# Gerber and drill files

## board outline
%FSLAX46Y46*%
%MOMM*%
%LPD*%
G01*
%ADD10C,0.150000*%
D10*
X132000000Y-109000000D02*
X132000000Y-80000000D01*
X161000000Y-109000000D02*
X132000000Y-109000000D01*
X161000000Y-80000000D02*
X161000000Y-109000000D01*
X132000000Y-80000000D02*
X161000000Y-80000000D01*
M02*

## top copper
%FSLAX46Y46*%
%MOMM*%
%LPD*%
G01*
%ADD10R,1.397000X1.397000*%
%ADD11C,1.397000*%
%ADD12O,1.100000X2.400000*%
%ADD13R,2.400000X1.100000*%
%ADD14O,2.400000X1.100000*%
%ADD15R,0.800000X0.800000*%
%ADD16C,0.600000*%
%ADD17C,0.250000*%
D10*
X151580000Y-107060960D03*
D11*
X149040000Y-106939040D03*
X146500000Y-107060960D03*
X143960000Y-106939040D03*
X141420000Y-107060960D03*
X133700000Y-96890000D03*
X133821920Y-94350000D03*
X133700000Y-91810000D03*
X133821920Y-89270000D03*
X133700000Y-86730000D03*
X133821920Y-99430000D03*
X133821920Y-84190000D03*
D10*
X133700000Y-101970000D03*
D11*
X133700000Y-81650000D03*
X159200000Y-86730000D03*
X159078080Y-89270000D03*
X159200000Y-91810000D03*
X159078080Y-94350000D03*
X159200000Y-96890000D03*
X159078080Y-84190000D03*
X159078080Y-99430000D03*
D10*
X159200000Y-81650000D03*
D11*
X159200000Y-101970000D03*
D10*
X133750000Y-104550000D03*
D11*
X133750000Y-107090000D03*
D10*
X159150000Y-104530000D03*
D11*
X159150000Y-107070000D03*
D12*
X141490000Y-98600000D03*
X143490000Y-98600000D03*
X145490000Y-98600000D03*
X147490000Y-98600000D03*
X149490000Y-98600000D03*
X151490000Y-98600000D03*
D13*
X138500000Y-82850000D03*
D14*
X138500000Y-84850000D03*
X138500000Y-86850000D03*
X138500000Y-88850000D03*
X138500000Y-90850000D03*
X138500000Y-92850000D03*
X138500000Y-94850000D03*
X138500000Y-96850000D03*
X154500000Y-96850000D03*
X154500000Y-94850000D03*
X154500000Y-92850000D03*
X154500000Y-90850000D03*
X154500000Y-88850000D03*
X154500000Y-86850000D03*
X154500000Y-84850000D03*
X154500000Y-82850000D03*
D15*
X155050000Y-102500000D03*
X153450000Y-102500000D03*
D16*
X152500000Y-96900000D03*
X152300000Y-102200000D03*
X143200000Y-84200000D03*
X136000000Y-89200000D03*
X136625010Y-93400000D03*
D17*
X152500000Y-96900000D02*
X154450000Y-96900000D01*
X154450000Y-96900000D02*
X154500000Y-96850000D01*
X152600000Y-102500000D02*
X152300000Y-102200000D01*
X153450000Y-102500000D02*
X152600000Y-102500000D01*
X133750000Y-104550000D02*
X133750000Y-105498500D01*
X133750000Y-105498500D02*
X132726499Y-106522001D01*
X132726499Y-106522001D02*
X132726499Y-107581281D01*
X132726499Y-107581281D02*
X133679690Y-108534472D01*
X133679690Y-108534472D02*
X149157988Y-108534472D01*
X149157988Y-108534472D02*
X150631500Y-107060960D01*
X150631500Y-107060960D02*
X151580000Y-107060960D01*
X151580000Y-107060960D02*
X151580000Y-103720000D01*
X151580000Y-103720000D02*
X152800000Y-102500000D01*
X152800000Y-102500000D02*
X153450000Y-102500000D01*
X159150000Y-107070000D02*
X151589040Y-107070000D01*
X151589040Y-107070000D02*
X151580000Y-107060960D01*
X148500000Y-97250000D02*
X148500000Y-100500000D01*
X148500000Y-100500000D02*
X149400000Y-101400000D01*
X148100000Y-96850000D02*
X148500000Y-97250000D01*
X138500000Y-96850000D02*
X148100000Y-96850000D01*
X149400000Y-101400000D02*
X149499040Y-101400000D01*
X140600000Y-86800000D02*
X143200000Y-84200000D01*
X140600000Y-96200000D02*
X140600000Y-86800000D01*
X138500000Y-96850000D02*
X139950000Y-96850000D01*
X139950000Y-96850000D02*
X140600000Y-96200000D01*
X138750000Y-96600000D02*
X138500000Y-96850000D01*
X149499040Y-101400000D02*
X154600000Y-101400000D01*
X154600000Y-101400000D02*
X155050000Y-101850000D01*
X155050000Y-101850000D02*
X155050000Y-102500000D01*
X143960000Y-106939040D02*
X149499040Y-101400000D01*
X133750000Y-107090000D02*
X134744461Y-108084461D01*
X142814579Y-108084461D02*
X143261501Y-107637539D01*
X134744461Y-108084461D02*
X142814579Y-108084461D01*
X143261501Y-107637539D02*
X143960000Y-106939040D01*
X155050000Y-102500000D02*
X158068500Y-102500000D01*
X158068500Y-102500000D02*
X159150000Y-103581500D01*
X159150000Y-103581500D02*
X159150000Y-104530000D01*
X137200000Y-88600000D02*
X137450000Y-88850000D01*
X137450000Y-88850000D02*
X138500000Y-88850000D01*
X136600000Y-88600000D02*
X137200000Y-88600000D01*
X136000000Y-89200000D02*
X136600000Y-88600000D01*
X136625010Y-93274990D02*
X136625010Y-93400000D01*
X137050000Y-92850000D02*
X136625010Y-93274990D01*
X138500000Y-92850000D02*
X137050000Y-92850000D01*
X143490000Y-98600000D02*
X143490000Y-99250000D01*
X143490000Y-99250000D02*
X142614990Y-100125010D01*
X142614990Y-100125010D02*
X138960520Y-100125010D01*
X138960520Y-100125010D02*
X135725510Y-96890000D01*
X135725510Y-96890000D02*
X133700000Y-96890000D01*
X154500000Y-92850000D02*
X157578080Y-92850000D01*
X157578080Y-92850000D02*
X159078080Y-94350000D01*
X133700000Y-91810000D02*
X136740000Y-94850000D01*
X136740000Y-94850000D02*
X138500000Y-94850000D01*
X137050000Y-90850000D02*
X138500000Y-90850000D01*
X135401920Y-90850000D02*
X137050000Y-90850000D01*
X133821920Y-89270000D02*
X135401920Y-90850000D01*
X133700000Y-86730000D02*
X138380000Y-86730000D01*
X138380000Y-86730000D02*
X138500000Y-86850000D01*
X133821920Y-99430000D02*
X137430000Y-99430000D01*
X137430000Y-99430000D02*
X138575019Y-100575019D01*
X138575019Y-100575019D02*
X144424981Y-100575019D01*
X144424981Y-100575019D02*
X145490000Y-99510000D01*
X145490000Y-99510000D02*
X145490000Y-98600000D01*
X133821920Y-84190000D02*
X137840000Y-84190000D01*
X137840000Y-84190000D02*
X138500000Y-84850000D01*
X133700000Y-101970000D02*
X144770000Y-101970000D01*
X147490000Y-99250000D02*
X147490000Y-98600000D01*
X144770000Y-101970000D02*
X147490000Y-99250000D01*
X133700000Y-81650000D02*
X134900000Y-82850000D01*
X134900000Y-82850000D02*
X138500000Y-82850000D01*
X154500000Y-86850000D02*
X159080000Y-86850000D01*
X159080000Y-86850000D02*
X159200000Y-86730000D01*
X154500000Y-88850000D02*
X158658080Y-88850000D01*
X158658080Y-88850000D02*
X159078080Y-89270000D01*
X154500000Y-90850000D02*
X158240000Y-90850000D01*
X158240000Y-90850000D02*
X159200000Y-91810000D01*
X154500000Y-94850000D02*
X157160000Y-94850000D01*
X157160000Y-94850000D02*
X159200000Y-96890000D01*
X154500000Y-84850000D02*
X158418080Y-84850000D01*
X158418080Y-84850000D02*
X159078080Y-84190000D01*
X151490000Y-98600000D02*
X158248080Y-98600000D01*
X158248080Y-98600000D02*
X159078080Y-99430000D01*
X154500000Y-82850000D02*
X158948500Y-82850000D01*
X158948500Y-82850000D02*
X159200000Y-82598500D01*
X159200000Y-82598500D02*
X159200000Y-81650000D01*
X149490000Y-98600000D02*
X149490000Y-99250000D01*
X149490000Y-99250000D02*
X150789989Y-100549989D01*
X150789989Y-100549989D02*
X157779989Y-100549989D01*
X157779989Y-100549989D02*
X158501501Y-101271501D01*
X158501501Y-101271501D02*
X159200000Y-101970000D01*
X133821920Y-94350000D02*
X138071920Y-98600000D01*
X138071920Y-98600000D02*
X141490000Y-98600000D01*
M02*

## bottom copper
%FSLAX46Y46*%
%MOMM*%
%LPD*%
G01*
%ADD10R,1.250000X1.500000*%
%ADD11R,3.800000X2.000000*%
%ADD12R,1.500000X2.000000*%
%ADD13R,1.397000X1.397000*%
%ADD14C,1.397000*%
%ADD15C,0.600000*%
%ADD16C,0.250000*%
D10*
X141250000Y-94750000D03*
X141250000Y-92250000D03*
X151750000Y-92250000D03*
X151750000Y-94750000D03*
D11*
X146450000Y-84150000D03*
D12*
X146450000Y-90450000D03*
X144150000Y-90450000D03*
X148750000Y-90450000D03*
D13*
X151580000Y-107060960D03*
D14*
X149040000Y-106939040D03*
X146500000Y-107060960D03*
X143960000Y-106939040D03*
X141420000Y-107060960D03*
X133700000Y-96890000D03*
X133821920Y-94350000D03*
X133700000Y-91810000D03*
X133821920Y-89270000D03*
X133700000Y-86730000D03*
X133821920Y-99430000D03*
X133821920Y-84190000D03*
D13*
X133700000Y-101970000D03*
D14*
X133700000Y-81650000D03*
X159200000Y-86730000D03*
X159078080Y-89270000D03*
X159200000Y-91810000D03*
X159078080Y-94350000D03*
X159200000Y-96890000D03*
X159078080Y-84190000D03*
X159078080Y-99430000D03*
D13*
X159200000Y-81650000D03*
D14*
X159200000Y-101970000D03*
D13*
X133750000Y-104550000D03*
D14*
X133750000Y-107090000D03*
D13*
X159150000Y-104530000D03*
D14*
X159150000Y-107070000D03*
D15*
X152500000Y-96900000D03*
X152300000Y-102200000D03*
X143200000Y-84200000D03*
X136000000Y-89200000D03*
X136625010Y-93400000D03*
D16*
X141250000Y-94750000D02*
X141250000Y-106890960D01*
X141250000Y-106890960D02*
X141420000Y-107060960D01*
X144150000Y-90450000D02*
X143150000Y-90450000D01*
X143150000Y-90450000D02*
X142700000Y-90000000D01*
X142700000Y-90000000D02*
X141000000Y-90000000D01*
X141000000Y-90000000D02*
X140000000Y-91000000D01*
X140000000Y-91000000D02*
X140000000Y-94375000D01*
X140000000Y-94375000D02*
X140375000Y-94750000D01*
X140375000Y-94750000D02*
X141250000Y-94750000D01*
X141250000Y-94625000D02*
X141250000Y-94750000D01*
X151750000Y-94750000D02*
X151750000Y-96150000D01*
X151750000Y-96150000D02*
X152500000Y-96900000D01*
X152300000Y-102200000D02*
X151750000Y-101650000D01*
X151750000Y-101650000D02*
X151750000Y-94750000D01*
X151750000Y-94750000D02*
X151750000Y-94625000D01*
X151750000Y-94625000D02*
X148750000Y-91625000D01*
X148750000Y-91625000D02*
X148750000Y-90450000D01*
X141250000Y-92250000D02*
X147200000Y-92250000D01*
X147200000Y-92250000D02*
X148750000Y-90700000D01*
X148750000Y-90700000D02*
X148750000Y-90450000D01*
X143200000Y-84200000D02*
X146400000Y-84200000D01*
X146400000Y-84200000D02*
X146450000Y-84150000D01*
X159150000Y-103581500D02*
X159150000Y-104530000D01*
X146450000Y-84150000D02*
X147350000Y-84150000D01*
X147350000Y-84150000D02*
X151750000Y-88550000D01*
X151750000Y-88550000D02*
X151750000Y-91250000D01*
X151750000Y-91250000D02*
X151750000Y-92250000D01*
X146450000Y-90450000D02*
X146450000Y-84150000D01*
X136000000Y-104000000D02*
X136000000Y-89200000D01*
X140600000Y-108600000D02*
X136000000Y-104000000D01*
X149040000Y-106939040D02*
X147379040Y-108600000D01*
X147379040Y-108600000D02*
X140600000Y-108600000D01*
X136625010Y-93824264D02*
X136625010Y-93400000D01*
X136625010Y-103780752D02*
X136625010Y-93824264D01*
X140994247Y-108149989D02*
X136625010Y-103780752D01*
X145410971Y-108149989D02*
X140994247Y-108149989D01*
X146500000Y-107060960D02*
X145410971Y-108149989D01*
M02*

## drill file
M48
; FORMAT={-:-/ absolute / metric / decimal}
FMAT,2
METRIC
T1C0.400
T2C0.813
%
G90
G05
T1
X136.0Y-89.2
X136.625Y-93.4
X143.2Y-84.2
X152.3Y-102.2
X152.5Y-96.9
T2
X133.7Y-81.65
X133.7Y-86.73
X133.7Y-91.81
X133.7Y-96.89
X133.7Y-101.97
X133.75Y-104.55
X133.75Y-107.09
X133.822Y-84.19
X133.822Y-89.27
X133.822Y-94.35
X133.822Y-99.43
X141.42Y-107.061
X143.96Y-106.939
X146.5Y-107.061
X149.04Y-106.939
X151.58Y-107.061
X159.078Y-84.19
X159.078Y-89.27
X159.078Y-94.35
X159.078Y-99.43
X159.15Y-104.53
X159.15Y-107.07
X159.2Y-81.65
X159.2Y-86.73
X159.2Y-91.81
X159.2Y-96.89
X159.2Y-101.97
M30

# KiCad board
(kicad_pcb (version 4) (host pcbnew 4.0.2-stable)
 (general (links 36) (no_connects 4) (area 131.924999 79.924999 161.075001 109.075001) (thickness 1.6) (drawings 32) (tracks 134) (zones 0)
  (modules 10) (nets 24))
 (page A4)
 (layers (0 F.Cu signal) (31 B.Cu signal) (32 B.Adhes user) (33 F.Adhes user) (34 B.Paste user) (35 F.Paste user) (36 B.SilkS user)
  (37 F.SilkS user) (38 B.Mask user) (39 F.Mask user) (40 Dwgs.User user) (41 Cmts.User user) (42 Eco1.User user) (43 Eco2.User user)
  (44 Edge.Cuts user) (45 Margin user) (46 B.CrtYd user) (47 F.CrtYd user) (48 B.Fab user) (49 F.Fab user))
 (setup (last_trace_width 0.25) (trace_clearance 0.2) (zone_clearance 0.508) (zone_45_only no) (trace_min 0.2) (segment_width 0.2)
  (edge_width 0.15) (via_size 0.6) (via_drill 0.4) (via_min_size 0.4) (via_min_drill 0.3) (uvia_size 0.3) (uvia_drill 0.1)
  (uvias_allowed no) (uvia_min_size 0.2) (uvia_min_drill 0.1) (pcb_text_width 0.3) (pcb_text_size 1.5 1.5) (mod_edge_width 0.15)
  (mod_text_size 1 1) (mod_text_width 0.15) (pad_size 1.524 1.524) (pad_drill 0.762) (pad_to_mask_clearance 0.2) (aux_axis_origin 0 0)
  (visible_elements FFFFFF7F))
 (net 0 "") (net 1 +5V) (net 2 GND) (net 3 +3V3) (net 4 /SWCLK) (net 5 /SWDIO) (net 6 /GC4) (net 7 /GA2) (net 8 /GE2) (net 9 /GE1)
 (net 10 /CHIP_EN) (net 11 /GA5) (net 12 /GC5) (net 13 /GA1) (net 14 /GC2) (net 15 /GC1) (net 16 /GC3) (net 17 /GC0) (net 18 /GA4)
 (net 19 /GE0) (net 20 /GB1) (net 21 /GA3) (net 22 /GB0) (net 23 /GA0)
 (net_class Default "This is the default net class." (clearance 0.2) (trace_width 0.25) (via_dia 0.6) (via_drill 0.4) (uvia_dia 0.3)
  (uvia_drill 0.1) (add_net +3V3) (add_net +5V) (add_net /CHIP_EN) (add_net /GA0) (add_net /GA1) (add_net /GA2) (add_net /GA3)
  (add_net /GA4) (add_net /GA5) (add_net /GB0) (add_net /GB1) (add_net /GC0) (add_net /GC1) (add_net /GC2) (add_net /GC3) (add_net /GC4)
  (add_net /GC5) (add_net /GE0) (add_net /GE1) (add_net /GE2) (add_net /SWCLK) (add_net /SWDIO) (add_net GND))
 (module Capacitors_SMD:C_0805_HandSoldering (layer B.Cu) (at 141.25 93.5 90)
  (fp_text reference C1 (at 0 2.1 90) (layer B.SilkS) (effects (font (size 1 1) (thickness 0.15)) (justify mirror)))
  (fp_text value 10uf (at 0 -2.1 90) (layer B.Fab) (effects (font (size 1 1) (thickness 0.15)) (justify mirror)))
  (pad 1 smd rect (at -1.25 0 90) (size 1.5 1.25) (layers B.Cu B.Paste B.Mask) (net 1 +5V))
  (pad 2 smd rect (at 1.25 0 90) (size 1.5 1.25) (layers B.Cu B.Paste B.Mask) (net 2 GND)))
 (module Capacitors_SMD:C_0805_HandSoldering (layer B.Cu) (at 151.75 93.5 270)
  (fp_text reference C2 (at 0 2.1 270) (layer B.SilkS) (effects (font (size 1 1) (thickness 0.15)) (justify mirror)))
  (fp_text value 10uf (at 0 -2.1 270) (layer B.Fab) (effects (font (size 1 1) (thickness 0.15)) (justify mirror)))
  (pad 1 smd rect (at -1.25 0 270) (size 1.5 1.25) (layers B.Cu B.Paste B.Mask) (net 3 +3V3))
  (pad 2 smd rect (at 1.25 0 270) (size 1.5 1.25) (layers B.Cu B.Paste B.Mask) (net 2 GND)))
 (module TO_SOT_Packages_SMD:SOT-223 (layer B.Cu) (at 146.45 87.3 90)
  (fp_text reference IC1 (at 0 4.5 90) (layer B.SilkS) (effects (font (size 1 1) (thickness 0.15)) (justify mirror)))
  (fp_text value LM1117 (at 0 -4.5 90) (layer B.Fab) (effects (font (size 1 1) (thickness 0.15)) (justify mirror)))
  (pad 4 smd rect (at 3.15 0 90) (size 2 3.8) (layers B.Cu B.Paste B.Mask) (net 3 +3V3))
  (pad 2 smd rect (at -3.15 0 90) (size 2 1.5) (layers B.Cu B.Paste B.Mask) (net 3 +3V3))
  (pad 3 smd rect (at -3.15 -2.3 90) (size 2 1.5) (layers B.Cu B.Paste B.Mask) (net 1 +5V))
  (pad 1 smd rect (at -3.15 2.3 90) (size 2 1.5) (layers B.Cu B.Paste B.Mask) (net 2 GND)))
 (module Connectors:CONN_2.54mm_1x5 (layer F.Cu) (at 146.5 107)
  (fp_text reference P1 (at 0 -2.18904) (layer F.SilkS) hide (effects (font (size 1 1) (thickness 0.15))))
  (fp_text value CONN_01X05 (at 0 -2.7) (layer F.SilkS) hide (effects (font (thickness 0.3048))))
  (pad 1 thru_hole rect (at 5.08 0.06096) (size 1.397 1.397) (drill 0.8128) (layers *.Cu *.Mask F.SilkS) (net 2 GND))
  (pad 2 thru_hole circle (at 2.54 -0.06096) (size 1.397 1.397) (drill 0.8128) (layers *.Cu *.Mask F.SilkS) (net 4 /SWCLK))
  (pad 3 thru_hole circle (at 0 0.06096) (size 1.397 1.397) (drill 0.8128) (layers *.Cu *.Mask F.SilkS) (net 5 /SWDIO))
  (pad 4 thru_hole circle (at -2.54 -0.06096) (size 1.397 1.397) (drill 0.8128) (layers *.Cu *.Mask F.SilkS) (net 3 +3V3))
  (pad 5 thru_hole circle (at -5.08 0.06096) (size 1.397 1.397) (drill 0.8128) (layers *.Cu *.Mask F.SilkS) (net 1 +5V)))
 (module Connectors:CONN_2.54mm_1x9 (layer F.Cu) (at 133.76096 91.81 270)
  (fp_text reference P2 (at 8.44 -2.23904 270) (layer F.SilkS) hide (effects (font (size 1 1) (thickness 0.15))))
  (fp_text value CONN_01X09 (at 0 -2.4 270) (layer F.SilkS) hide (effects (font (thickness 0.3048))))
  (pad 3 thru_hole circle (at 5.08 0.06096 270) (size 1.397 1.397) (drill 0.8128) (layers *.Cu *.Mask F.SilkS) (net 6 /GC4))
  (pad 4 thru_hole circle (at 2.54 -0.06096 270) (size 1.397 1.397) (drill 0.8128) (layers *.Cu *.Mask F.SilkS) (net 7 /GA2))
  (pad 5 thru_hole circle (at 0 0.06096 270) (size 1.397 1.397) (drill 0.8128) (layers *.Cu *.Mask F.SilkS) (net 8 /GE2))
  (pad 6 thru_hole circle (at -2.54 -0.06096 270) (size 1.397 1.397) (drill 0.8128) (layers *.Cu *.Mask F.SilkS) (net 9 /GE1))
  (pad 7 thru_hole circle (at -5.08 0.06096 270) (size 1.397 1.397) (drill 0.8128) (layers *.Cu *.Mask F.SilkS) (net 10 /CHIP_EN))
  (pad 2 thru_hole circle (at 7.62 -0.06096 270) (size 1.397 1.397) (drill 0.8128) (layers *.Cu *.Mask F.SilkS) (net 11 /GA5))
  (pad 8 thru_hole circle (at -7.62 -0.06096 270) (size 1.397 1.397) (drill 0.8128) (layers *.Cu *.Mask F.SilkS) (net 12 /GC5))
  (pad 1 thru_hole rect (at 10.16 0.06096 270) (size 1.397 1.397) (drill 0.8128) (layers *.Cu *.Mask F.SilkS) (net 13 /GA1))
  (pad 9 thru_hole circle (at -10.16 0.06096 270) (size 1.397 1.397) (drill 0.8128) (layers *.Cu *.Mask F.SilkS) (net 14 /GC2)))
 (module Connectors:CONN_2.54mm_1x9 (layer F.Cu) (at 159.13904 91.81 90)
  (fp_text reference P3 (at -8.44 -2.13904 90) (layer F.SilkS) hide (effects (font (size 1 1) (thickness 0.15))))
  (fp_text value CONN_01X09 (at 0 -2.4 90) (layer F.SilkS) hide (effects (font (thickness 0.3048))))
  (pad 3 thru_hole circle (at 5.08 0.06096 90) (size 1.397 1.397) (drill 0.8128) (layers *.Cu *.Mask F.SilkS) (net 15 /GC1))
  (pad 4 thru_hole circle (at 2.54 -0.06096 90) (size 1.397 1.397) (drill 0.8128) (layers *.Cu *.Mask F.SilkS) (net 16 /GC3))
  (pad 5 thru_hole circle (at 0 0.06096 90) (size 1.397 1.397) (drill 0.8128) (layers *.Cu *.Mask F.SilkS) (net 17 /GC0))
  (pad 6 thru_hole circle (at -2.54 -0.06096 90) (size 1.397 1.397) (drill 0.8128) (layers *.Cu *.Mask F.SilkS) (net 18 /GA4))
  (pad 7 thru_hole circle (at -5.08 0.06096 90) (size 1.397 1.397) (drill 0.8128) (layers *.Cu *.Mask F.SilkS) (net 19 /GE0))
  (pad 2 thru_hole circle (at 7.62 -0.06096 90) (size 1.397 1.397) (drill 0.8128) (layers *.Cu *.Mask F.SilkS) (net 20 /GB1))
  (pad 8 thru_hole circle (at -7.62 -0.06096 90) (size 1.397 1.397) (drill 0.8128) (layers *.Cu *.Mask F.SilkS) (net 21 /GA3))
  (pad 1 thru_hole rect (at 10.16 0.06096 90) (size 1.397 1.397) (drill 0.8128) (layers *.Cu *.Mask F.SilkS) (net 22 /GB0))
  (pad 9 thru_hole circle (at -10.16 0.06096 90) (size 1.397 1.397) (drill 0.8128) (layers *.Cu *.Mask F.SilkS) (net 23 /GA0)))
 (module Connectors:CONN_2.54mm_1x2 (layer F.Cu) (at 133.75 105.82 90)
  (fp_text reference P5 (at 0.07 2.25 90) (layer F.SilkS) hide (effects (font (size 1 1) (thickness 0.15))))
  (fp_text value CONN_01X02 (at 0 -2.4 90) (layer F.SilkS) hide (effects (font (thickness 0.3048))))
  (pad 1 thru_hole rect (at 1.27 0 90) (size 1.397 1.397) (drill 0.8128) (layers *.Cu *.Mask F.SilkS) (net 2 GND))
  (pad 2 thru_hole circle (at -1.27 0 90) (size 1.397 1.397) (drill 0.8128) (layers *.Cu *.Mask F.SilkS) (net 3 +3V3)))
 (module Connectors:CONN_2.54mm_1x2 (layer F.Cu) (at 159.15 105.8 90)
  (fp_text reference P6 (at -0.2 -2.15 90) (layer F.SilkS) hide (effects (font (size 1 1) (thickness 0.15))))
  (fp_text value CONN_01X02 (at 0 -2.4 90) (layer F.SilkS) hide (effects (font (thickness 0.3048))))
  (pad 1 thru_hole rect (at 1.27 0 90) (size 1.397 1.397) (drill 0.8128) (layers *.Cu *.Mask F.SilkS) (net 3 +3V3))
  (pad 2 thru_hole circle (at -1.27 0 90) (size 1.397 1.397) (drill 0.8128) (layers *.Cu *.Mask F.SilkS) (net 2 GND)))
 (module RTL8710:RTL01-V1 (layer F.Cu) (at 138.5 82.85)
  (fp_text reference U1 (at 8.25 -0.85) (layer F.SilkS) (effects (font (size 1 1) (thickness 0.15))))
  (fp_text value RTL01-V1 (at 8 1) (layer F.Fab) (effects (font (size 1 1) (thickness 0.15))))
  (pad 9 smd oval (at 2.99 15.75 90) (size 2.4 1.1) (layers F.Cu F.Paste F.Mask) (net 7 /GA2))
  (pad 10 smd oval (at 4.99 15.75 90) (size 2.4 1.1) (layers F.Cu F.Paste F.Mask) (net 6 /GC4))
  (pad 11 smd oval (at 6.99 15.75 90) (size 2.4 1.1) (layers F.Cu F.Paste F.Mask) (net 11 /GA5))
  (pad 12 smd oval (at 8.99 15.75 90) (size 2.4 1.1) (layers F.Cu F.Paste F.Mask) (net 13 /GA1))
  (pad 13 smd oval (at 10.99 15.75 90) (size 2.4 1.1) (layers F.Cu F.Paste F.Mask) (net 23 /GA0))
  (pad 14 smd oval (at 12.99 15.75 90) (size 2.4 1.1) (layers F.Cu F.Paste F.Mask) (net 21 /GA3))
  (pad 1 smd rect (at 0 0) (size 2.4 1.1) (layers F.Cu F.Paste F.Mask) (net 14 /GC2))
  (pad 2 smd oval (at 0 2) (size 2.4 1.1) (layers F.Cu F.Paste F.Mask) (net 12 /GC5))
  (pad 3 smd oval (at 0 4) (size 2.4 1.1) (layers F.Cu F.Paste F.Mask) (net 10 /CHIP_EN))
  (pad 4 smd oval (at 0 6) (size 2.4 1.1) (layers F.Cu F.Paste F.Mask) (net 4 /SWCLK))
  (pad 5 smd oval (at 0 8) (size 2.4 1.1) (layers F.Cu F.Paste F.Mask) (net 9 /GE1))
  (pad 6 smd oval (at 0 10) (size 2.4 1.1) (layers F.Cu F.Paste F.Mask) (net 5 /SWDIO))
  (pad 7 smd oval (at 0 12) (size 2.4 1.1) (layers F.Cu F.Paste F.Mask) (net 8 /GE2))
  (pad 8 smd oval (at 0 14) (size 2.4 1.1) (layers F.Cu F.Paste F.Mask) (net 3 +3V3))
  (pad 15 smd oval (at 16 14) (size 2.4 1.1) (layers F.Cu F.Paste F.Mask) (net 2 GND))
  (pad 16 smd oval (at 16 12) (size 2.4 1.1) (layers F.Cu F.Paste F.Mask) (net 19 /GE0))
  (pad 17 smd oval (at 16 10) (size 2.4 1.1) (layers F.Cu F.Paste F.Mask) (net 18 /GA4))
  (pad 18 smd oval (at 16 8) (size 2.4 1.1) (layers F.Cu F.Paste F.Mask) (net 17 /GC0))
  (pad 19 smd oval (at 16 6) (size 2.4 1.1) (layers F.Cu F.Paste F.Mask) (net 16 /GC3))
  (pad 20 smd oval (at 16 4) (size 2.4 1.1) (layers F.Cu F.Paste F.Mask) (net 15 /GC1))
  (pad 21 smd oval (at 16 2) (size 2.4 1.1) (layers F.Cu F.Paste F.Mask) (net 20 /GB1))
  (pad 22 smd oval (at 16 0) (size 2.4 1.1) (layers F.Cu F.Paste F.Mask) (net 22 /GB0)))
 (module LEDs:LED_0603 (layer F.Cu) (at 154.25 102.5)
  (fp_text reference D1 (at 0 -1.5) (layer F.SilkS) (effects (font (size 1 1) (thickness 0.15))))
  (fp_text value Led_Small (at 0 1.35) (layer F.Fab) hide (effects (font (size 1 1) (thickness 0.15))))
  (pad 2 smd rect (at 0.8 0 180) (size 0.8 0.8) (layers F.Cu F.Paste F.Mask) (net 3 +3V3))
  (pad 1 smd rect (at -0.8 0 180) (size 0.8 0.8) (layers F.Cu F.Paste F.Mask) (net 2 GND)))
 (gr_line (start 132 109) (end 132 80) (layer Edge.Cuts) (width 0.15))
 (gr_line (start 161 109) (end 132 109) (layer Edge.Cuts) (width 0.15))
 (gr_line (start 161 80) (end 161 109) (layer Edge.Cuts) (width 0.15))
 (gr_line (start 132 80) (end 161 80) (layer Edge.Cuts) (width 0.15))
 (segment (start 141.25 94.75) (end 141.25 106.89096) (width 0.25) (layer B.Cu) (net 1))
 (segment (start 141.25 106.89096) (end 141.42 107.06096) (width 0.25) (layer B.Cu) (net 1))
 (segment (start 144.15 90.45) (end 143.15 90.45) (width 0.25) (layer B.Cu) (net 1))
 (segment (start 143.15 90.45) (end 142.7 90) (width 0.25) (layer B.Cu) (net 1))
 (segment (start 142.7 90) (end 141 90) (width 0.25) (layer B.Cu) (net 1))
 (segment (start 141 90) (end 140 91) (width 0.25) (layer B.Cu) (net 1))
 (segment (start 140 91) (end 140 94.375) (width 0.25) (layer B.Cu) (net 1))
 (segment (start 140 94.375) (end 140.375 94.75) (width 0.25) (layer B.Cu) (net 1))
 (segment (start 140.375 94.75) (end 141.25 94.75) (width 0.25) (layer B.Cu) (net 1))
 (segment (start 141.25 94.625) (end 141.25 94.75) (width 0.25) (layer B.Cu) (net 1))
 (segment (start 152.5 96.9) (end 154.45 96.9) (width 0.25) (layer F.Cu) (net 2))
 (segment (start 154.45 96.9) (end 154.5 96.85) (width 0.25) (layer F.Cu) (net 2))
 (segment (start 151.75 94.75) (end 151.75 96.15) (width 0.25) (layer B.Cu) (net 2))
 (segment (start 151.75 96.15) (end 152.5 96.9) (width 0.25) (layer B.Cu) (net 2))
 (via (at 152.5 96.9) (size 0.6) (drill 0.4) (layers F.Cu B.Cu) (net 2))
 (segment (start 152.3 102.2) (end 151.75 101.65) (width 0.25) (layer B.Cu) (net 2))
 (segment (start 151.75 101.65) (end 151.75 94.75) (width 0.25) (layer B.Cu) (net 2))
 (segment (start 152.6 102.5) (end 152.3 102.2) (width 0.25) (layer F.Cu) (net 2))
 (via (at 152.3 102.2) (size 0.6) (drill 0.4) (layers F.Cu B.Cu) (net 2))
 (segment (start 153.45 102.5) (end 152.6 102.5) (width 0.25) (layer F.Cu) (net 2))
 (segment (start 151.75 94.75) (end 151.75 94.625) (width 0.25) (layer B.Cu) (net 2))
 (segment (start 151.75 94.625) (end 148.75 91.625) (width 0.25) (layer B.Cu) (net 2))
 (segment (start 148.75 91.625) (end 148.75 90.45) (width 0.25) (layer B.Cu) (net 2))
 (segment (start 141.25 92.25) (end 147.2 92.25) (width 0.25) (layer B.Cu) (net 2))
 (segment (start 147.2 92.25) (end 148.75 90.7) (width 0.25) (layer B.Cu) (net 2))
 (segment (start 148.75 90.7) (end 148.75 90.45) (width 0.25) (layer B.Cu) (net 2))
 (segment (start 133.75 104.55) (end 133.75 105.4985) (width 0.25) (layer F.Cu) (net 2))
 (segment (start 133.75 105.4985) (end 132.726499 106.522001) (width 0.25) (layer F.Cu) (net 2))
 (segment (start 132.726499 106.522001) (end 132.726499 107.581281) (width 0.25) (layer F.Cu) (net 2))
 (segment (start 132.726499 107.581281) (end 133.67969 108.534472) (width 0.25) (layer F.Cu) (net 2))
 (segment (start 133.67969 108.534472) (end 149.157988 108.534472) (width 0.25) (layer F.Cu) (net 2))
 (segment (start 149.157988 108.534472) (end 150.6315 107.06096) (width 0.25) (layer F.Cu) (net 2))
 (segment (start 150.6315 107.06096) (end 151.58 107.06096) (width 0.25) (layer F.Cu) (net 2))
 (segment (start 151.58 107.06096) (end 151.58 103.72) (width 0.25) (layer F.Cu) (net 2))
 (segment (start 151.58 103.72) (end 152.8 102.5) (width 0.25) (layer F.Cu) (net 2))
 (segment (start 152.8 102.5) (end 153.45 102.5) (width 0.25) (layer F.Cu) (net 2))
 (segment (start 159.15 107.07) (end 151.58904 107.07) (width 0.25) (layer F.Cu) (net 2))
 (segment (start 151.58904 107.07) (end 151.58 107.06096) (width 0.25) (layer F.Cu) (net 2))
 (segment (start 148.5 97.25) (end 148.5 100.5) (width 0.25) (layer F.Cu) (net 3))
 (segment (start 148.5 100.5) (end 149.4 101.4) (width 0.25) (layer F.Cu) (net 3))
 (segment (start 148.1 96.85) (end 148.5 97.25) (width 0.25) (layer F.Cu) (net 3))
 (segment (start 138.5 96.85) (end 148.1 96.85) (width 0.25) (layer F.Cu) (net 3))
 (segment (start 149.4 101.4) (end 149.49904 101.4) (width 0.25) (layer F.Cu) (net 3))
 (segment (start 143.2 84.2) (end 146.4 84.2) (width 0.25) (layer B.Cu) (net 3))
 (segment (start 146.4 84.2) (end 146.45 84.15) (width 0.25) (layer B.Cu) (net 3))
 (segment (start 140.6 86.8) (end 143.2 84.2) (width 0.25) (layer F.Cu) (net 3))
 (via (at 143.2 84.2) (size 0.6) (drill 0.4) (layers F.Cu B.Cu) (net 3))
 (segment (start 140.6 96.2) (end 140.6 86.8) (width 0.25) (layer F.Cu) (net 3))
 (segment (start 138.5 96.85) (end 139.95 96.85) (width 0.25) (layer F.Cu) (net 3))
 (segment (start 139.95 96.85) (end 140.6 96.2) (width 0.25) (layer F.Cu) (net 3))
 (segment (start 159.15 103.5815) (end 159.15 104.53) (width 0.25) (layer B.Cu) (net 3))
 (segment (start 138.75 96.6) (end 138.5 96.85) (width 0.25) (layer F.Cu) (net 3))
 (segment (start 149.49904 101.4) (end 154.6 101.4) (width 0.25) (layer F.Cu) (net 3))
 (segment (start 154.6 101.4) (end 155.05 101.85) (width 0.25) (layer F.Cu) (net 3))
 (segment (start 155.05 101.85) (end 155.05 102.5) (width 0.25) (layer F.Cu) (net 3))
 (segment (start 143.96 106.93904) (end 149.49904 101.4) (width 0.25) (layer F.Cu) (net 3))
 (segment (start 146.45 84.15) (end 147.35 84.15) (width 0.25) (layer B.Cu) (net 3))
 (segment (start 147.35 84.15) (end 151.75 88.55) (width 0.25) (layer B.Cu) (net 3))
 (segment (start 151.75 88.55) (end 151.75 91.25) (width 0.25) (layer B.Cu) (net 3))
 (segment (start 151.75 91.25) (end 151.75 92.25) (width 0.25) (layer B.Cu) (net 3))
 (segment (start 146.45 90.45) (end 146.45 84.15) (width 0.25) (layer B.Cu) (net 3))
 (segment (start 133.75 107.09) (end 134.744461 108.084461) (width 0.25) (layer F.Cu) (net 3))
 (segment (start 142.814579 108.084461) (end 143.261501 107.637539) (width 0.25) (layer F.Cu) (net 3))
 (segment (start 134.744461 108.084461) (end 142.814579 108.084461) (width 0.25) (layer F.Cu) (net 3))
 (segment (start 143.261501 107.637539) (end 143.96 106.93904) (width 0.25) (layer F.Cu) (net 3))
 (segment (start 155.05 102.5) (end 158.0685 102.5) (width 0.25) (layer F.Cu) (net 3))
 (segment (start 158.0685 102.5) (end 159.15 103.5815) (width 0.25) (layer F.Cu) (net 3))
 (segment (start 159.15 103.5815) (end 159.15 104.53) (width 0.25) (layer F.Cu) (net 3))
 (segment (start 137.2 88.6) (end 137.45 88.85) (width 0.25) (layer F.Cu) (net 4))
 (segment (start 137.45 88.85) (end 138.5 88.85) (width 0.25) (layer F.Cu) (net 4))
 (segment (start 136.6 88.6) (end 137.2 88.6) (width 0.25) (layer F.Cu) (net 4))
 (segment (start 136 89.2) (end 136.6 88.6) (width 0.25) (layer F.Cu) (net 4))
 (segment (start 136 104) (end 136 89.2) (width 0.25) (layer B.Cu) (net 4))
 (via (at 136 89.2) (size 0.6) (drill 0.4) (layers F.Cu B.Cu) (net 4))
 (segment (start 140.6 108.6) (end 136 104) (width 0.25) (layer B.Cu) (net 4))
 (segment (start 149.04 106.93904) (end 147.37904 108.6) (width 0.25) (layer B.Cu) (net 4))
 (segment (start 147.37904 108.6) (end 140.6 108.6) (width 0.25) (layer B.Cu) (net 4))
 (segment (start 136.62501 93.824264) (end 136.62501 93.4) (width 0.25) (layer B.Cu) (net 5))
 (segment (start 136.62501 103.780752) (end 136.62501 93.824264) (width 0.25) (layer B.Cu) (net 5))
 (segment (start 140.994247 108.149989) (end 136.62501 103.780752) (width 0.25) (layer B.Cu) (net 5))
 (segment (start 145.410971 108.149989) (end 140.994247 108.149989) (width 0.25) (layer B.Cu) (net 5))
 (segment (start 146.5 107.06096) (end 145.410971 108.149989) (width 0.25) (layer B.Cu) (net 5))
 (segment (start 136.62501 93.27499) (end 136.62501 93.4) (width 0.25) (layer F.Cu) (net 5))
 (segment (start 137.05 92.85) (end 136.62501 93.27499) (width 0.25) (layer F.Cu) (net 5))
 (segment (start 138.5 92.85) (end 137.05 92.85) (width 0.25) (layer F.Cu) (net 5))
 (via (at 136.62501 93.4) (size 0.6) (drill 0.4) (layers F.Cu B.Cu) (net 5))
 (segment (start 143.49 98.6) (end 143.49 99.25) (width 0.25) (layer F.Cu) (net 6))
 (segment (start 143.49 99.25) (end 142.61499 100.12501) (width 0.25) (layer F.Cu) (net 6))
 (segment (start 142.61499 100.12501) (end 138.96052 100.12501) (width 0.25) (layer F.Cu) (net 6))
 (segment (start 138.96052 100.12501) (end 135.72551 96.89) (width 0.25) (layer F.Cu) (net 6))
 (segment (start 135.72551 96.89) (end 133.7 96.89) (width 0.25) (layer F.Cu) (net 6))
 (segment (start 154.5 92.85) (end 157.57808 92.85) (width 0.25) (layer F.Cu) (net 18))
 (segment (start 157.57808 92.85) (end 159.07808 94.35) (width 0.25) (layer F.Cu) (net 18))
 (segment (start 133.7 91.81) (end 136.74 94.85) (width 0.25) (layer F.Cu) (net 8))
 (segment (start 136.74 94.85) (end 138.5 94.85) (width 0.25) (layer F.Cu) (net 8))
 (segment (start 137.05 90.85) (end 138.5 90.85) (width 0.25) (layer F.Cu) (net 9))
 (segment (start 135.40192 90.85) (end 137.05 90.85) (width 0.25) (layer F.Cu) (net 9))
 (segment (start 133.82192 89.27) (end 135.40192 90.85) (width 0.25) (layer F.Cu) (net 9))
 (segment (start 133.7 86.73) (end 138.38 86.73) (width 0.25) (layer F.Cu) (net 10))
 (segment (start 138.38 86.73) (end 138.5 86.85) (width 0.25) (layer F.Cu) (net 10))
 (segment (start 133.82192 99.43) (end 137.43 99.43) (width 0.25) (layer F.Cu) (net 11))
 (segment (start 137.43 99.43) (end 138.575019 100.575019) (width 0.25) (layer F.Cu) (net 11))
 (segment (start 138.575019 100.575019) (end 144.424981 100.575019) (width 0.25) (layer F.Cu) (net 11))
 (segment (start 144.424981 100.575019) (end 145.49 99.51) (width 0.25) (layer F.Cu) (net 11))
 (segment (start 145.49 99.51) (end 145.49 98.6) (width 0.25) (layer F.Cu) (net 11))
 (segment (start 133.82192 84.19) (end 137.84 84.19) (width 0.25) (layer F.Cu) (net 12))
 (segment (start 137.84 84.19) (end 138.5 84.85) (width 0.25) (layer F.Cu) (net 12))
 (segment (start 133.7 101.97) (end 144.77 101.97) (width 0.25) (layer F.Cu) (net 13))
 (segment (start 147.49 99.25) (end 147.49 98.6) (width 0.25) (layer F.Cu) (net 13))
 (segment (start 144.77 101.97) (end 147.49 99.25) (width 0.25) (layer F.Cu) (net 13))
 (segment (start 133.7 81.65) (end 134.9 82.85) (width 0.25) (layer F.Cu) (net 14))
 (segment (start 134.9 82.85) (end 138.5 82.85) (width 0.25) (layer F.Cu) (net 14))
 (segment (start 154.5 86.85) (end 159.08 86.85) (width 0.25) (layer F.Cu) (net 15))
 (segment (start 159.08 86.85) (end 159.2 86.73) (width 0.25) (layer F.Cu) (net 15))
 (segment (start 154.5 88.85) (end 158.65808 88.85) (width 0.25) (layer F.Cu) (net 16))
 (segment (start 158.65808 88.85) (end 159.07808 89.27) (width 0.25) (layer F.Cu) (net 16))
 (segment (start 154.5 90.85) (end 158.24 90.85) (width 0.25) (layer F.Cu) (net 17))
 (segment (start 158.24 90.85) (end 159.2 91.81) (width 0.25) (layer F.Cu) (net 17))
 (segment (start 154.5 94.85) (end 157.16 94.85) (width 0.25) (layer F.Cu) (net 19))
 (segment (start 157.16 94.85) (end 159.2 96.89) (width 0.25) (layer F.Cu) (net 19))
 (segment (start 154.5 84.85) (end 158.41808 84.85) (width 0.25) (layer F.Cu) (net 20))
 (segment (start 158.41808 84.85) (end 159.07808 84.19) (width 0.25) (layer F.Cu) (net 20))
 (segment (start 151.49 98.6) (end 158.24808 98.6) (width 0.25) (layer F.Cu) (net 21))
 (segment (start 158.24808 98.6) (end 159.07808 99.43) (width 0.25) (layer F.Cu) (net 21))
 (segment (start 154.5 82.85) (end 158.9485 82.85) (width 0.25) (layer F.Cu) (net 22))
 (segment (start 158.9485 82.85) (end 159.2 82.5985) (width 0.25) (layer F.Cu) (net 22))
 (segment (start 159.2 82.5985) (end 159.2 81.65) (width 0.25) (layer F.Cu) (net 22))
 (segment (start 149.49 98.6) (end 149.49 99.25) (width 0.25) (layer F.Cu) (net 23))
 (segment (start 149.49 99.25) (end 150.789989 100.549989) (width 0.25) (layer F.Cu) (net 23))
 (segment (start 150.789989 100.549989) (end 157.779989 100.549989) (width 0.25) (layer F.Cu) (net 23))
 (segment (start 157.779989 100.549989) (end 158.501501 101.271501) (width 0.25) (layer F.Cu) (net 23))
 (segment (start 158.501501 101.271501) (end 159.2 101.97) (width 0.25) (layer F.Cu) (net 23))
 (segment (start 133.82192 94.35) (end 138.07192 98.6) (width 0.25) (layer F.Cu) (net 7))
 (segment (start 138.07192 98.6) (end 141.49 98.6) (width 0.25) (layer F.Cu) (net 7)))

